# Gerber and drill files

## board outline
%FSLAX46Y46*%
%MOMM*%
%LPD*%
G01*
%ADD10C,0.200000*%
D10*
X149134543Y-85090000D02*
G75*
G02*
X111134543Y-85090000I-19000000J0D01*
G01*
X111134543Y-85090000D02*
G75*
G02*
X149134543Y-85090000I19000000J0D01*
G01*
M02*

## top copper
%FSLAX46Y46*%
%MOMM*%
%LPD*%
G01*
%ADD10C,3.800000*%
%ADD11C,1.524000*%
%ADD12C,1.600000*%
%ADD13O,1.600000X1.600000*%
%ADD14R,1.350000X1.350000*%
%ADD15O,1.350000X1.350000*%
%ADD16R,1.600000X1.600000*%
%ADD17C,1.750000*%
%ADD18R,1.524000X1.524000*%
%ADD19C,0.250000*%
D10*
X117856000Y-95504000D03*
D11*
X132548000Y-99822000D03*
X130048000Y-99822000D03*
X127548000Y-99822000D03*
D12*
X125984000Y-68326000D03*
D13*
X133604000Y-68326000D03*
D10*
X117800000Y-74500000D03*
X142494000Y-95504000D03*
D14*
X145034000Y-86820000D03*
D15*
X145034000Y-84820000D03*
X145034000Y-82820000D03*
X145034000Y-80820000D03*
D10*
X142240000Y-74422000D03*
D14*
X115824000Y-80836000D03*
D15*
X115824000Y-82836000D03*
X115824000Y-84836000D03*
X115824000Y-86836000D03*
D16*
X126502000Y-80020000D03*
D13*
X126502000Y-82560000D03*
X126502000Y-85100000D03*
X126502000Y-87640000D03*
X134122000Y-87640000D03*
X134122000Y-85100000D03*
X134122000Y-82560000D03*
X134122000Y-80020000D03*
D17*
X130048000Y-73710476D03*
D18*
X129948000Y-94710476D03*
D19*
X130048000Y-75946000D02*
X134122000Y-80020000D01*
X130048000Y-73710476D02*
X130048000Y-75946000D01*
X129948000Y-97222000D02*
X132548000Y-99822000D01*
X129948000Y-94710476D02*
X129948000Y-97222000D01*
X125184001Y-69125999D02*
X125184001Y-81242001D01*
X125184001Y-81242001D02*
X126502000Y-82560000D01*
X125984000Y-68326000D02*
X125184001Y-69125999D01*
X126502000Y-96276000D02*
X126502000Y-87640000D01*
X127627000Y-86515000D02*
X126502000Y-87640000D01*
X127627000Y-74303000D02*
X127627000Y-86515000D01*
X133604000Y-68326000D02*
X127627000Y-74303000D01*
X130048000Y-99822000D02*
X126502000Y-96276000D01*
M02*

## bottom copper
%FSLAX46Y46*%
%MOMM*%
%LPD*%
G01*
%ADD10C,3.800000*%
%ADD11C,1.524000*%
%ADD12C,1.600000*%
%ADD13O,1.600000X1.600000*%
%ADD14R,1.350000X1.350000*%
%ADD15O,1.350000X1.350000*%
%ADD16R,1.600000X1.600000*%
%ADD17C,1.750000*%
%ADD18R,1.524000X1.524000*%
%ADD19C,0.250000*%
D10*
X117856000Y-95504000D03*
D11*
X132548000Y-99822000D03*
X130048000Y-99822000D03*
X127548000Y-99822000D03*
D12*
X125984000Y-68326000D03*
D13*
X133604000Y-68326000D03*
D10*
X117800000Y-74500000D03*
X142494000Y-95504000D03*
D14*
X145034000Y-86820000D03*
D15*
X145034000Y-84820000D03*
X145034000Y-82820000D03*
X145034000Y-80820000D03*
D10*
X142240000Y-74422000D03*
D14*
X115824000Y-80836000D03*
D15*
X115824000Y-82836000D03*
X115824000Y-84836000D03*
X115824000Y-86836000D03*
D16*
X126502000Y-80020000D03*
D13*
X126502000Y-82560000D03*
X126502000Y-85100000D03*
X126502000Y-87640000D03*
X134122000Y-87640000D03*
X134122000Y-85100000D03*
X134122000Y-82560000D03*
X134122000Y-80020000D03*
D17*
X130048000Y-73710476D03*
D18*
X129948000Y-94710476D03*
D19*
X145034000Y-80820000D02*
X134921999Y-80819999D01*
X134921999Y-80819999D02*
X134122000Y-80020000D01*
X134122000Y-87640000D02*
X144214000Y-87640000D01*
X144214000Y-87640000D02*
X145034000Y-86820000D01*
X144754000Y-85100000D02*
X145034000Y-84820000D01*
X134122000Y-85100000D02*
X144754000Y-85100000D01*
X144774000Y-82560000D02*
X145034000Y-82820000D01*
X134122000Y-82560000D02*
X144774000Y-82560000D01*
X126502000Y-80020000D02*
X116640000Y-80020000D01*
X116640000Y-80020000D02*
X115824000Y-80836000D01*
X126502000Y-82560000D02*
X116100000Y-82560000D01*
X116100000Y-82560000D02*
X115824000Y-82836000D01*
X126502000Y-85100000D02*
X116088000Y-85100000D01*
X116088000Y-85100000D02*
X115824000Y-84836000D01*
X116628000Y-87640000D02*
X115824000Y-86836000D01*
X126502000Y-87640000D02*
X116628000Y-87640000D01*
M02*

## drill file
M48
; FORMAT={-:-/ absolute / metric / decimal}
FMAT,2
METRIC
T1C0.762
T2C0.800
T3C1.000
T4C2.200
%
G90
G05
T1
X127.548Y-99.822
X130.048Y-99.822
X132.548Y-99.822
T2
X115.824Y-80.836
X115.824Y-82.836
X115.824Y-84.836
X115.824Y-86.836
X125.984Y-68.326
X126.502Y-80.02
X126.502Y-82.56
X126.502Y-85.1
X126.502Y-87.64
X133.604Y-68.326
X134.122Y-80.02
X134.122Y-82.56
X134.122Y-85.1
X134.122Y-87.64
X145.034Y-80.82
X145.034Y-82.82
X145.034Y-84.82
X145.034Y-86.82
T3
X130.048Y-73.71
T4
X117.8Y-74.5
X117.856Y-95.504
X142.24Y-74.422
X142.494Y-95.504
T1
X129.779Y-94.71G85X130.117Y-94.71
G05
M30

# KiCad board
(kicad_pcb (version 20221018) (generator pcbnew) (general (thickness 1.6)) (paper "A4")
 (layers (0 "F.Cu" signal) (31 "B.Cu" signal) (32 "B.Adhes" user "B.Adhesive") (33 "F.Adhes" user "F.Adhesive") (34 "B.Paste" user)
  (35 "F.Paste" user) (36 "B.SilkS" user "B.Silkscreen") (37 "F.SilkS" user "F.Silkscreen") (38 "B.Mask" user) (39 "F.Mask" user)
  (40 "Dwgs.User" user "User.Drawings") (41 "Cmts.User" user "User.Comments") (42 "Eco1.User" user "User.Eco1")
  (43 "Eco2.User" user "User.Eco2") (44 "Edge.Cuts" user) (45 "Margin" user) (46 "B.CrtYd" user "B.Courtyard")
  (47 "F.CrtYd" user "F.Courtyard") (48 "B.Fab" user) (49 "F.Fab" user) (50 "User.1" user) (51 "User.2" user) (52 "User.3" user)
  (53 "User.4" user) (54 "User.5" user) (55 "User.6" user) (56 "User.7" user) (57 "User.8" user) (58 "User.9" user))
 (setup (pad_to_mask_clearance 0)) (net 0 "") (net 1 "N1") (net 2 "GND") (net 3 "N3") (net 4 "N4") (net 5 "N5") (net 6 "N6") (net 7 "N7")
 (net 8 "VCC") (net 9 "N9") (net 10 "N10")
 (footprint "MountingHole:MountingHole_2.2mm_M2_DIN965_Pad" (layer "F.Cu") (at 117.856 95.504)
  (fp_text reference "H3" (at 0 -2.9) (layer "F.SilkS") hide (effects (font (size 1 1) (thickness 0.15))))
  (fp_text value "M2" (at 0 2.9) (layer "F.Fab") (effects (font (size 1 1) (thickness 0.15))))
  (pad "1" thru_hole circle (at 0 0) (size 3.8 3.8) (drill 2.2) (layers "*.Cu" "*.Mask")))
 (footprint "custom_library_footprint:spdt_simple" (layer "F.Cu") (at 126.548 99.822 -90)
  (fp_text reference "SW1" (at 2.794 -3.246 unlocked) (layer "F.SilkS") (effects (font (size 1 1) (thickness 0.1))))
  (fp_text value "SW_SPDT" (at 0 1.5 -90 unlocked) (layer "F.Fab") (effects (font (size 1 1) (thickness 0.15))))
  (pad "1" thru_hole circle (at 0 -6 270) (size 1.524 1.524) (drill 0.762) (layers "*.Cu" "*.Mask") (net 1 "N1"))
  (pad "2" thru_hole circle (at 0 -3.5 270) (size 1.524 1.524) (drill 0.762) (layers "*.Cu" "*.Mask") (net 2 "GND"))
  (pad "3" thru_hole circle (at 0 -1 270) (size 1.524 1.524) (drill 0.762) (layers "*.Cu" "*.Mask") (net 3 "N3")))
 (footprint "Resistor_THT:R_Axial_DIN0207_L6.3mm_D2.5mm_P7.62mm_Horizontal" (layer "F.Cu") (at 125.984 68.326)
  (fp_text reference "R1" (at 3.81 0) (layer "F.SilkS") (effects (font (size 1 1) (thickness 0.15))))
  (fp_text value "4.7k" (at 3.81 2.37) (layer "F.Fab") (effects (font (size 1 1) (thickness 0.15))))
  (pad "1" thru_hole circle (at 0 0) (size 1.6 1.6) (drill 0.8) (layers "*.Cu" "*.Mask") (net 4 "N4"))
  (pad "2" thru_hole oval (at 7.62 0) (size 1.6 1.6) (drill 0.8) (layers "*.Cu" "*.Mask") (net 2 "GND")))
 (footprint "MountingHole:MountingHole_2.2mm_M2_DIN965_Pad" (layer "F.Cu") (at 117.8 74.5)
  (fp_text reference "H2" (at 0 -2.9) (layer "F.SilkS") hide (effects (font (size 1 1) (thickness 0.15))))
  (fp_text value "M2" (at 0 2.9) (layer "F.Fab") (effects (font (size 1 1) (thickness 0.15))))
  (pad "1" thru_hole circle (at 0 0) (size 3.8 3.8) (drill 2.2) (layers "*.Cu" "*.Mask")))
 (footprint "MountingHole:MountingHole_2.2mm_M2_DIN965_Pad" (layer "F.Cu") (at 142.494 95.504)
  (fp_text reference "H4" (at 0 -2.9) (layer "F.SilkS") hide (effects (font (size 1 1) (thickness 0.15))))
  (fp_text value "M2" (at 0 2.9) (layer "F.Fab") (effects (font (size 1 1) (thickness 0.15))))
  (pad "1" thru_hole circle (at 0 0) (size 3.8 3.8) (drill 2.2) (layers "*.Cu" "*.Mask")))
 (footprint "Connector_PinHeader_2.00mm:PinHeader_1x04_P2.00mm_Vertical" (layer "F.Cu") (at 145.034 86.82 180)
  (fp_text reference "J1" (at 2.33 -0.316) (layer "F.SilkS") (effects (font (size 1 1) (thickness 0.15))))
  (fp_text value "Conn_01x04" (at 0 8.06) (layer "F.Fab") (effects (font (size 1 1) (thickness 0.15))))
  (pad "1" thru_hole rect (at 0 0 180) (size 1.35 1.35) (drill 0.8) (layers "*.Cu" "*.Mask") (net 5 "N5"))
  (pad "2" thru_hole oval (at 0 2 180) (size 1.35 1.35) (drill 0.8) (layers "*.Cu" "*.Mask") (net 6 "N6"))
  (pad "3" thru_hole oval (at 0 4 180) (size 1.35 1.35) (drill 0.8) (layers "*.Cu" "*.Mask") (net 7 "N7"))
  (pad "4" thru_hole oval (at 0 6 180) (size 1.35 1.35) (drill 0.8) (layers "*.Cu" "*.Mask") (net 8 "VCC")))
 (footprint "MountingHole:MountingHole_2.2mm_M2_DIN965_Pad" (layer "F.Cu") (at 142.24 74.422)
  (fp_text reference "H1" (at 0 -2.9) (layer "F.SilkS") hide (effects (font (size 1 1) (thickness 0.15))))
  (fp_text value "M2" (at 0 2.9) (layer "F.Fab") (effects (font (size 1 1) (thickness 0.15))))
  (pad "1" thru_hole circle (at 0 0) (size 3.8 3.8) (drill 2.2) (layers "*.Cu" "*.Mask")))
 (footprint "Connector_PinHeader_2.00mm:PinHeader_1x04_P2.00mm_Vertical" (layer "F.Cu") (at 115.824 80.836)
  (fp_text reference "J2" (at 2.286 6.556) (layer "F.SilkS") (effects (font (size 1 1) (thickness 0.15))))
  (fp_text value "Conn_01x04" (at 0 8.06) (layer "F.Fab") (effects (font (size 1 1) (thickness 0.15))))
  (pad "1" thru_hole rect (at 0 0) (size 1.35 1.35) (drill 0.8) (layers "*.Cu" "*.Mask") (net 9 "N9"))
  (pad "2" thru_hole oval (at 0 2) (size 1.35 1.35) (drill 0.8) (layers "*.Cu" "*.Mask") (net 4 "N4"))
  (pad "3" thru_hole oval (at 0 4) (size 1.35 1.35) (drill 0.8) (layers "*.Cu" "*.Mask") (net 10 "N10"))
  (pad "4" thru_hole oval (at 0 6) (size 1.35 1.35) (drill 0.8) (layers "*.Cu" "*.Mask") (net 2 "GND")))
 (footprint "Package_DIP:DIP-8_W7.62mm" (layer "F.Cu") (at 126.502 80.02)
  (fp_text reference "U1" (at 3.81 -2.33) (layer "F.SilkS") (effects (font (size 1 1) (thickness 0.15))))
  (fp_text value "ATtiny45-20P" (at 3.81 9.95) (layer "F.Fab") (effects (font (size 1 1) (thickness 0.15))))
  (pad "1" thru_hole rect (at 0 0) (size 1.6 1.6) (drill 0.8) (layers "*.Cu" "*.Mask") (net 9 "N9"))
  (pad "2" thru_hole oval (at 0 2.54) (size 1.6 1.6) (drill 0.8) (layers "*.Cu" "*.Mask") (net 4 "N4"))
  (pad "3" thru_hole oval (at 0 5.08) (size 1.6 1.6) (drill 0.8) (layers "*.Cu" "*.Mask") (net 10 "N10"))
  (pad "4" thru_hole oval (at 0 7.62) (size 1.6 1.6) (drill 0.8) (layers "*.Cu" "*.Mask") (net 2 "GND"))
  (pad "5" thru_hole oval (at 7.62 7.62) (size 1.6 1.6) (drill 0.8) (layers "*.Cu" "*.Mask") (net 5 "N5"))
  (pad "6" thru_hole oval (at 7.62 5.08) (size 1.6 1.6) (drill 0.8) (layers "*.Cu" "*.Mask") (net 6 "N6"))
  (pad "7" thru_hole oval (at 7.62 2.54) (size 1.6 1.6) (drill 0.8) (layers "*.Cu" "*.Mask") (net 7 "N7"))
  (pad "8" thru_hole oval (at 7.62 0) (size 1.6 1.6) (drill 0.8) (layers "*.Cu" "*.Mask") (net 8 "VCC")))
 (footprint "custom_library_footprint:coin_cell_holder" (layer "B.Cu") (at 130.048 81.710476 90)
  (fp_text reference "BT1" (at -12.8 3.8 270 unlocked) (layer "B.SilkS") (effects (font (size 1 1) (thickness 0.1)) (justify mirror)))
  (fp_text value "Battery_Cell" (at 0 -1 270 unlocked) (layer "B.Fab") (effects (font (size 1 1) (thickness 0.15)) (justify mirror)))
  (pad "1" thru_hole circle (at 8 0 90) (size 1.75 1.75) (drill 1) (layers "*.Cu" "*.Mask") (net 8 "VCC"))
  (pad "2" thru_hole rect (at -13 -0.1 90) (size 1.524 1.524) (drill oval 0.762 1.1) (layers "*.Cu" "*.Mask") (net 1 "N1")))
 (gr_circle (center 130.134543 85.09) (end 149.134543 85.09) (stroke (width 0.2) (type default)) (fill none) (layer "Edge.Cuts"))
 (segment (start 130.048 75.946) (end 134.122 80.02) (width 0.25) (layer "F.Cu") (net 8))
 (segment (start 130.048 73.710476) (end 130.048 75.946) (width 0.25) (layer "F.Cu") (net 8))
 (segment (start 145.034 80.82) (end 134.921999 80.819999) (width 0.25) (layer "B.Cu") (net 8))
 (segment (start 134.921999 80.819999) (end 134.122 80.02) (width 0.25) (layer "B.Cu") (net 8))
 (segment (start 129.948 97.222) (end 132.548 99.822) (width 0.25) (layer "F.Cu") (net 1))
 (segment (start 129.948 94.710476) (end 129.948 97.222) (width 0.25) (layer "F.Cu") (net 1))
 (segment (start 134.122 87.64) (end 144.214 87.64) (width 0.25) (layer "B.Cu") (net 5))
 (segment (start 144.214 87.64) (end 145.034 86.82) (width 0.25) (layer "B.Cu") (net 5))
 (segment (start 144.754 85.1) (end 145.034 84.82) (width 0.25) (layer "B.Cu") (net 6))
 (segment (start 134.122 85.1) (end 144.754 85.1) (width 0.25) (layer "B.Cu") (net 6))
 (segment (start 144.774 82.56) (end 145.034 82.82) (width 0.25) (layer "B.Cu") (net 7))
 (segment (start 134.122 82.56) (end 144.774 82.56) (width 0.25) (layer "B.Cu") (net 7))
 (segment (start 126.502 80.02) (end 116.64 80.02) (width 0.25) (layer "B.Cu") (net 9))
 (segment (start 116.64 80.02) (end 115.824 80.836) (width 0.25) (layer "B.Cu") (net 9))
 (segment (start 125.184001 69.125999) (end 125.184001 81.242001) (width 0.25) (layer "F.Cu") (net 4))
 (segment (start 125.184001 81.242001) (end 126.502 82.56) (width 0.25) (layer "F.Cu") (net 4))
 (segment (start 125.984 68.326) (end 125.184001 69.125999) (width 0.25) (layer "F.Cu") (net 4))
 (segment (start 126.502 82.56) (end 116.1 82.56) (width 0.25) (layer "B.Cu") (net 4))
 (segment (start 116.1 82.56) (end 115.824 82.836) (width 0.25) (layer "B.Cu") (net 4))
 (segment (start 126.502 85.1) (end 116.088 85.1) (width 0.25) (layer "B.Cu") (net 10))
 (segment (start 116.088 85.1) (end 115.824 84.836) (width 0.25) (layer "B.Cu") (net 10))
 (segment (start 126.502 96.276) (end 126.502 87.64) (width 0.25) (layer "F.Cu") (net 2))
 (segment (start 127.627 86.515) (end 126.502 87.64) (width 0.25) (layer "F.Cu") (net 2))
 (segment (start 127.627 74.303) (end 127.627 86.515) (width 0.25) (layer "F.Cu") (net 2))
 (segment (start 133.604 68.326) (end 127.627 74.303) (width 0.25) (layer "F.Cu") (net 2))
 (segment (start 130.048 99.822) (end 126.502 96.276) (width 0.25) (layer "F.Cu") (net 2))
 (segment (start 116.628 87.64) (end 115.824 86.836) (width 0.25) (layer "B.Cu") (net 2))
 (segment (start 126.502 87.64) (end 116.628 87.64) (width 0.25) (layer "B.Cu") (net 2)))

